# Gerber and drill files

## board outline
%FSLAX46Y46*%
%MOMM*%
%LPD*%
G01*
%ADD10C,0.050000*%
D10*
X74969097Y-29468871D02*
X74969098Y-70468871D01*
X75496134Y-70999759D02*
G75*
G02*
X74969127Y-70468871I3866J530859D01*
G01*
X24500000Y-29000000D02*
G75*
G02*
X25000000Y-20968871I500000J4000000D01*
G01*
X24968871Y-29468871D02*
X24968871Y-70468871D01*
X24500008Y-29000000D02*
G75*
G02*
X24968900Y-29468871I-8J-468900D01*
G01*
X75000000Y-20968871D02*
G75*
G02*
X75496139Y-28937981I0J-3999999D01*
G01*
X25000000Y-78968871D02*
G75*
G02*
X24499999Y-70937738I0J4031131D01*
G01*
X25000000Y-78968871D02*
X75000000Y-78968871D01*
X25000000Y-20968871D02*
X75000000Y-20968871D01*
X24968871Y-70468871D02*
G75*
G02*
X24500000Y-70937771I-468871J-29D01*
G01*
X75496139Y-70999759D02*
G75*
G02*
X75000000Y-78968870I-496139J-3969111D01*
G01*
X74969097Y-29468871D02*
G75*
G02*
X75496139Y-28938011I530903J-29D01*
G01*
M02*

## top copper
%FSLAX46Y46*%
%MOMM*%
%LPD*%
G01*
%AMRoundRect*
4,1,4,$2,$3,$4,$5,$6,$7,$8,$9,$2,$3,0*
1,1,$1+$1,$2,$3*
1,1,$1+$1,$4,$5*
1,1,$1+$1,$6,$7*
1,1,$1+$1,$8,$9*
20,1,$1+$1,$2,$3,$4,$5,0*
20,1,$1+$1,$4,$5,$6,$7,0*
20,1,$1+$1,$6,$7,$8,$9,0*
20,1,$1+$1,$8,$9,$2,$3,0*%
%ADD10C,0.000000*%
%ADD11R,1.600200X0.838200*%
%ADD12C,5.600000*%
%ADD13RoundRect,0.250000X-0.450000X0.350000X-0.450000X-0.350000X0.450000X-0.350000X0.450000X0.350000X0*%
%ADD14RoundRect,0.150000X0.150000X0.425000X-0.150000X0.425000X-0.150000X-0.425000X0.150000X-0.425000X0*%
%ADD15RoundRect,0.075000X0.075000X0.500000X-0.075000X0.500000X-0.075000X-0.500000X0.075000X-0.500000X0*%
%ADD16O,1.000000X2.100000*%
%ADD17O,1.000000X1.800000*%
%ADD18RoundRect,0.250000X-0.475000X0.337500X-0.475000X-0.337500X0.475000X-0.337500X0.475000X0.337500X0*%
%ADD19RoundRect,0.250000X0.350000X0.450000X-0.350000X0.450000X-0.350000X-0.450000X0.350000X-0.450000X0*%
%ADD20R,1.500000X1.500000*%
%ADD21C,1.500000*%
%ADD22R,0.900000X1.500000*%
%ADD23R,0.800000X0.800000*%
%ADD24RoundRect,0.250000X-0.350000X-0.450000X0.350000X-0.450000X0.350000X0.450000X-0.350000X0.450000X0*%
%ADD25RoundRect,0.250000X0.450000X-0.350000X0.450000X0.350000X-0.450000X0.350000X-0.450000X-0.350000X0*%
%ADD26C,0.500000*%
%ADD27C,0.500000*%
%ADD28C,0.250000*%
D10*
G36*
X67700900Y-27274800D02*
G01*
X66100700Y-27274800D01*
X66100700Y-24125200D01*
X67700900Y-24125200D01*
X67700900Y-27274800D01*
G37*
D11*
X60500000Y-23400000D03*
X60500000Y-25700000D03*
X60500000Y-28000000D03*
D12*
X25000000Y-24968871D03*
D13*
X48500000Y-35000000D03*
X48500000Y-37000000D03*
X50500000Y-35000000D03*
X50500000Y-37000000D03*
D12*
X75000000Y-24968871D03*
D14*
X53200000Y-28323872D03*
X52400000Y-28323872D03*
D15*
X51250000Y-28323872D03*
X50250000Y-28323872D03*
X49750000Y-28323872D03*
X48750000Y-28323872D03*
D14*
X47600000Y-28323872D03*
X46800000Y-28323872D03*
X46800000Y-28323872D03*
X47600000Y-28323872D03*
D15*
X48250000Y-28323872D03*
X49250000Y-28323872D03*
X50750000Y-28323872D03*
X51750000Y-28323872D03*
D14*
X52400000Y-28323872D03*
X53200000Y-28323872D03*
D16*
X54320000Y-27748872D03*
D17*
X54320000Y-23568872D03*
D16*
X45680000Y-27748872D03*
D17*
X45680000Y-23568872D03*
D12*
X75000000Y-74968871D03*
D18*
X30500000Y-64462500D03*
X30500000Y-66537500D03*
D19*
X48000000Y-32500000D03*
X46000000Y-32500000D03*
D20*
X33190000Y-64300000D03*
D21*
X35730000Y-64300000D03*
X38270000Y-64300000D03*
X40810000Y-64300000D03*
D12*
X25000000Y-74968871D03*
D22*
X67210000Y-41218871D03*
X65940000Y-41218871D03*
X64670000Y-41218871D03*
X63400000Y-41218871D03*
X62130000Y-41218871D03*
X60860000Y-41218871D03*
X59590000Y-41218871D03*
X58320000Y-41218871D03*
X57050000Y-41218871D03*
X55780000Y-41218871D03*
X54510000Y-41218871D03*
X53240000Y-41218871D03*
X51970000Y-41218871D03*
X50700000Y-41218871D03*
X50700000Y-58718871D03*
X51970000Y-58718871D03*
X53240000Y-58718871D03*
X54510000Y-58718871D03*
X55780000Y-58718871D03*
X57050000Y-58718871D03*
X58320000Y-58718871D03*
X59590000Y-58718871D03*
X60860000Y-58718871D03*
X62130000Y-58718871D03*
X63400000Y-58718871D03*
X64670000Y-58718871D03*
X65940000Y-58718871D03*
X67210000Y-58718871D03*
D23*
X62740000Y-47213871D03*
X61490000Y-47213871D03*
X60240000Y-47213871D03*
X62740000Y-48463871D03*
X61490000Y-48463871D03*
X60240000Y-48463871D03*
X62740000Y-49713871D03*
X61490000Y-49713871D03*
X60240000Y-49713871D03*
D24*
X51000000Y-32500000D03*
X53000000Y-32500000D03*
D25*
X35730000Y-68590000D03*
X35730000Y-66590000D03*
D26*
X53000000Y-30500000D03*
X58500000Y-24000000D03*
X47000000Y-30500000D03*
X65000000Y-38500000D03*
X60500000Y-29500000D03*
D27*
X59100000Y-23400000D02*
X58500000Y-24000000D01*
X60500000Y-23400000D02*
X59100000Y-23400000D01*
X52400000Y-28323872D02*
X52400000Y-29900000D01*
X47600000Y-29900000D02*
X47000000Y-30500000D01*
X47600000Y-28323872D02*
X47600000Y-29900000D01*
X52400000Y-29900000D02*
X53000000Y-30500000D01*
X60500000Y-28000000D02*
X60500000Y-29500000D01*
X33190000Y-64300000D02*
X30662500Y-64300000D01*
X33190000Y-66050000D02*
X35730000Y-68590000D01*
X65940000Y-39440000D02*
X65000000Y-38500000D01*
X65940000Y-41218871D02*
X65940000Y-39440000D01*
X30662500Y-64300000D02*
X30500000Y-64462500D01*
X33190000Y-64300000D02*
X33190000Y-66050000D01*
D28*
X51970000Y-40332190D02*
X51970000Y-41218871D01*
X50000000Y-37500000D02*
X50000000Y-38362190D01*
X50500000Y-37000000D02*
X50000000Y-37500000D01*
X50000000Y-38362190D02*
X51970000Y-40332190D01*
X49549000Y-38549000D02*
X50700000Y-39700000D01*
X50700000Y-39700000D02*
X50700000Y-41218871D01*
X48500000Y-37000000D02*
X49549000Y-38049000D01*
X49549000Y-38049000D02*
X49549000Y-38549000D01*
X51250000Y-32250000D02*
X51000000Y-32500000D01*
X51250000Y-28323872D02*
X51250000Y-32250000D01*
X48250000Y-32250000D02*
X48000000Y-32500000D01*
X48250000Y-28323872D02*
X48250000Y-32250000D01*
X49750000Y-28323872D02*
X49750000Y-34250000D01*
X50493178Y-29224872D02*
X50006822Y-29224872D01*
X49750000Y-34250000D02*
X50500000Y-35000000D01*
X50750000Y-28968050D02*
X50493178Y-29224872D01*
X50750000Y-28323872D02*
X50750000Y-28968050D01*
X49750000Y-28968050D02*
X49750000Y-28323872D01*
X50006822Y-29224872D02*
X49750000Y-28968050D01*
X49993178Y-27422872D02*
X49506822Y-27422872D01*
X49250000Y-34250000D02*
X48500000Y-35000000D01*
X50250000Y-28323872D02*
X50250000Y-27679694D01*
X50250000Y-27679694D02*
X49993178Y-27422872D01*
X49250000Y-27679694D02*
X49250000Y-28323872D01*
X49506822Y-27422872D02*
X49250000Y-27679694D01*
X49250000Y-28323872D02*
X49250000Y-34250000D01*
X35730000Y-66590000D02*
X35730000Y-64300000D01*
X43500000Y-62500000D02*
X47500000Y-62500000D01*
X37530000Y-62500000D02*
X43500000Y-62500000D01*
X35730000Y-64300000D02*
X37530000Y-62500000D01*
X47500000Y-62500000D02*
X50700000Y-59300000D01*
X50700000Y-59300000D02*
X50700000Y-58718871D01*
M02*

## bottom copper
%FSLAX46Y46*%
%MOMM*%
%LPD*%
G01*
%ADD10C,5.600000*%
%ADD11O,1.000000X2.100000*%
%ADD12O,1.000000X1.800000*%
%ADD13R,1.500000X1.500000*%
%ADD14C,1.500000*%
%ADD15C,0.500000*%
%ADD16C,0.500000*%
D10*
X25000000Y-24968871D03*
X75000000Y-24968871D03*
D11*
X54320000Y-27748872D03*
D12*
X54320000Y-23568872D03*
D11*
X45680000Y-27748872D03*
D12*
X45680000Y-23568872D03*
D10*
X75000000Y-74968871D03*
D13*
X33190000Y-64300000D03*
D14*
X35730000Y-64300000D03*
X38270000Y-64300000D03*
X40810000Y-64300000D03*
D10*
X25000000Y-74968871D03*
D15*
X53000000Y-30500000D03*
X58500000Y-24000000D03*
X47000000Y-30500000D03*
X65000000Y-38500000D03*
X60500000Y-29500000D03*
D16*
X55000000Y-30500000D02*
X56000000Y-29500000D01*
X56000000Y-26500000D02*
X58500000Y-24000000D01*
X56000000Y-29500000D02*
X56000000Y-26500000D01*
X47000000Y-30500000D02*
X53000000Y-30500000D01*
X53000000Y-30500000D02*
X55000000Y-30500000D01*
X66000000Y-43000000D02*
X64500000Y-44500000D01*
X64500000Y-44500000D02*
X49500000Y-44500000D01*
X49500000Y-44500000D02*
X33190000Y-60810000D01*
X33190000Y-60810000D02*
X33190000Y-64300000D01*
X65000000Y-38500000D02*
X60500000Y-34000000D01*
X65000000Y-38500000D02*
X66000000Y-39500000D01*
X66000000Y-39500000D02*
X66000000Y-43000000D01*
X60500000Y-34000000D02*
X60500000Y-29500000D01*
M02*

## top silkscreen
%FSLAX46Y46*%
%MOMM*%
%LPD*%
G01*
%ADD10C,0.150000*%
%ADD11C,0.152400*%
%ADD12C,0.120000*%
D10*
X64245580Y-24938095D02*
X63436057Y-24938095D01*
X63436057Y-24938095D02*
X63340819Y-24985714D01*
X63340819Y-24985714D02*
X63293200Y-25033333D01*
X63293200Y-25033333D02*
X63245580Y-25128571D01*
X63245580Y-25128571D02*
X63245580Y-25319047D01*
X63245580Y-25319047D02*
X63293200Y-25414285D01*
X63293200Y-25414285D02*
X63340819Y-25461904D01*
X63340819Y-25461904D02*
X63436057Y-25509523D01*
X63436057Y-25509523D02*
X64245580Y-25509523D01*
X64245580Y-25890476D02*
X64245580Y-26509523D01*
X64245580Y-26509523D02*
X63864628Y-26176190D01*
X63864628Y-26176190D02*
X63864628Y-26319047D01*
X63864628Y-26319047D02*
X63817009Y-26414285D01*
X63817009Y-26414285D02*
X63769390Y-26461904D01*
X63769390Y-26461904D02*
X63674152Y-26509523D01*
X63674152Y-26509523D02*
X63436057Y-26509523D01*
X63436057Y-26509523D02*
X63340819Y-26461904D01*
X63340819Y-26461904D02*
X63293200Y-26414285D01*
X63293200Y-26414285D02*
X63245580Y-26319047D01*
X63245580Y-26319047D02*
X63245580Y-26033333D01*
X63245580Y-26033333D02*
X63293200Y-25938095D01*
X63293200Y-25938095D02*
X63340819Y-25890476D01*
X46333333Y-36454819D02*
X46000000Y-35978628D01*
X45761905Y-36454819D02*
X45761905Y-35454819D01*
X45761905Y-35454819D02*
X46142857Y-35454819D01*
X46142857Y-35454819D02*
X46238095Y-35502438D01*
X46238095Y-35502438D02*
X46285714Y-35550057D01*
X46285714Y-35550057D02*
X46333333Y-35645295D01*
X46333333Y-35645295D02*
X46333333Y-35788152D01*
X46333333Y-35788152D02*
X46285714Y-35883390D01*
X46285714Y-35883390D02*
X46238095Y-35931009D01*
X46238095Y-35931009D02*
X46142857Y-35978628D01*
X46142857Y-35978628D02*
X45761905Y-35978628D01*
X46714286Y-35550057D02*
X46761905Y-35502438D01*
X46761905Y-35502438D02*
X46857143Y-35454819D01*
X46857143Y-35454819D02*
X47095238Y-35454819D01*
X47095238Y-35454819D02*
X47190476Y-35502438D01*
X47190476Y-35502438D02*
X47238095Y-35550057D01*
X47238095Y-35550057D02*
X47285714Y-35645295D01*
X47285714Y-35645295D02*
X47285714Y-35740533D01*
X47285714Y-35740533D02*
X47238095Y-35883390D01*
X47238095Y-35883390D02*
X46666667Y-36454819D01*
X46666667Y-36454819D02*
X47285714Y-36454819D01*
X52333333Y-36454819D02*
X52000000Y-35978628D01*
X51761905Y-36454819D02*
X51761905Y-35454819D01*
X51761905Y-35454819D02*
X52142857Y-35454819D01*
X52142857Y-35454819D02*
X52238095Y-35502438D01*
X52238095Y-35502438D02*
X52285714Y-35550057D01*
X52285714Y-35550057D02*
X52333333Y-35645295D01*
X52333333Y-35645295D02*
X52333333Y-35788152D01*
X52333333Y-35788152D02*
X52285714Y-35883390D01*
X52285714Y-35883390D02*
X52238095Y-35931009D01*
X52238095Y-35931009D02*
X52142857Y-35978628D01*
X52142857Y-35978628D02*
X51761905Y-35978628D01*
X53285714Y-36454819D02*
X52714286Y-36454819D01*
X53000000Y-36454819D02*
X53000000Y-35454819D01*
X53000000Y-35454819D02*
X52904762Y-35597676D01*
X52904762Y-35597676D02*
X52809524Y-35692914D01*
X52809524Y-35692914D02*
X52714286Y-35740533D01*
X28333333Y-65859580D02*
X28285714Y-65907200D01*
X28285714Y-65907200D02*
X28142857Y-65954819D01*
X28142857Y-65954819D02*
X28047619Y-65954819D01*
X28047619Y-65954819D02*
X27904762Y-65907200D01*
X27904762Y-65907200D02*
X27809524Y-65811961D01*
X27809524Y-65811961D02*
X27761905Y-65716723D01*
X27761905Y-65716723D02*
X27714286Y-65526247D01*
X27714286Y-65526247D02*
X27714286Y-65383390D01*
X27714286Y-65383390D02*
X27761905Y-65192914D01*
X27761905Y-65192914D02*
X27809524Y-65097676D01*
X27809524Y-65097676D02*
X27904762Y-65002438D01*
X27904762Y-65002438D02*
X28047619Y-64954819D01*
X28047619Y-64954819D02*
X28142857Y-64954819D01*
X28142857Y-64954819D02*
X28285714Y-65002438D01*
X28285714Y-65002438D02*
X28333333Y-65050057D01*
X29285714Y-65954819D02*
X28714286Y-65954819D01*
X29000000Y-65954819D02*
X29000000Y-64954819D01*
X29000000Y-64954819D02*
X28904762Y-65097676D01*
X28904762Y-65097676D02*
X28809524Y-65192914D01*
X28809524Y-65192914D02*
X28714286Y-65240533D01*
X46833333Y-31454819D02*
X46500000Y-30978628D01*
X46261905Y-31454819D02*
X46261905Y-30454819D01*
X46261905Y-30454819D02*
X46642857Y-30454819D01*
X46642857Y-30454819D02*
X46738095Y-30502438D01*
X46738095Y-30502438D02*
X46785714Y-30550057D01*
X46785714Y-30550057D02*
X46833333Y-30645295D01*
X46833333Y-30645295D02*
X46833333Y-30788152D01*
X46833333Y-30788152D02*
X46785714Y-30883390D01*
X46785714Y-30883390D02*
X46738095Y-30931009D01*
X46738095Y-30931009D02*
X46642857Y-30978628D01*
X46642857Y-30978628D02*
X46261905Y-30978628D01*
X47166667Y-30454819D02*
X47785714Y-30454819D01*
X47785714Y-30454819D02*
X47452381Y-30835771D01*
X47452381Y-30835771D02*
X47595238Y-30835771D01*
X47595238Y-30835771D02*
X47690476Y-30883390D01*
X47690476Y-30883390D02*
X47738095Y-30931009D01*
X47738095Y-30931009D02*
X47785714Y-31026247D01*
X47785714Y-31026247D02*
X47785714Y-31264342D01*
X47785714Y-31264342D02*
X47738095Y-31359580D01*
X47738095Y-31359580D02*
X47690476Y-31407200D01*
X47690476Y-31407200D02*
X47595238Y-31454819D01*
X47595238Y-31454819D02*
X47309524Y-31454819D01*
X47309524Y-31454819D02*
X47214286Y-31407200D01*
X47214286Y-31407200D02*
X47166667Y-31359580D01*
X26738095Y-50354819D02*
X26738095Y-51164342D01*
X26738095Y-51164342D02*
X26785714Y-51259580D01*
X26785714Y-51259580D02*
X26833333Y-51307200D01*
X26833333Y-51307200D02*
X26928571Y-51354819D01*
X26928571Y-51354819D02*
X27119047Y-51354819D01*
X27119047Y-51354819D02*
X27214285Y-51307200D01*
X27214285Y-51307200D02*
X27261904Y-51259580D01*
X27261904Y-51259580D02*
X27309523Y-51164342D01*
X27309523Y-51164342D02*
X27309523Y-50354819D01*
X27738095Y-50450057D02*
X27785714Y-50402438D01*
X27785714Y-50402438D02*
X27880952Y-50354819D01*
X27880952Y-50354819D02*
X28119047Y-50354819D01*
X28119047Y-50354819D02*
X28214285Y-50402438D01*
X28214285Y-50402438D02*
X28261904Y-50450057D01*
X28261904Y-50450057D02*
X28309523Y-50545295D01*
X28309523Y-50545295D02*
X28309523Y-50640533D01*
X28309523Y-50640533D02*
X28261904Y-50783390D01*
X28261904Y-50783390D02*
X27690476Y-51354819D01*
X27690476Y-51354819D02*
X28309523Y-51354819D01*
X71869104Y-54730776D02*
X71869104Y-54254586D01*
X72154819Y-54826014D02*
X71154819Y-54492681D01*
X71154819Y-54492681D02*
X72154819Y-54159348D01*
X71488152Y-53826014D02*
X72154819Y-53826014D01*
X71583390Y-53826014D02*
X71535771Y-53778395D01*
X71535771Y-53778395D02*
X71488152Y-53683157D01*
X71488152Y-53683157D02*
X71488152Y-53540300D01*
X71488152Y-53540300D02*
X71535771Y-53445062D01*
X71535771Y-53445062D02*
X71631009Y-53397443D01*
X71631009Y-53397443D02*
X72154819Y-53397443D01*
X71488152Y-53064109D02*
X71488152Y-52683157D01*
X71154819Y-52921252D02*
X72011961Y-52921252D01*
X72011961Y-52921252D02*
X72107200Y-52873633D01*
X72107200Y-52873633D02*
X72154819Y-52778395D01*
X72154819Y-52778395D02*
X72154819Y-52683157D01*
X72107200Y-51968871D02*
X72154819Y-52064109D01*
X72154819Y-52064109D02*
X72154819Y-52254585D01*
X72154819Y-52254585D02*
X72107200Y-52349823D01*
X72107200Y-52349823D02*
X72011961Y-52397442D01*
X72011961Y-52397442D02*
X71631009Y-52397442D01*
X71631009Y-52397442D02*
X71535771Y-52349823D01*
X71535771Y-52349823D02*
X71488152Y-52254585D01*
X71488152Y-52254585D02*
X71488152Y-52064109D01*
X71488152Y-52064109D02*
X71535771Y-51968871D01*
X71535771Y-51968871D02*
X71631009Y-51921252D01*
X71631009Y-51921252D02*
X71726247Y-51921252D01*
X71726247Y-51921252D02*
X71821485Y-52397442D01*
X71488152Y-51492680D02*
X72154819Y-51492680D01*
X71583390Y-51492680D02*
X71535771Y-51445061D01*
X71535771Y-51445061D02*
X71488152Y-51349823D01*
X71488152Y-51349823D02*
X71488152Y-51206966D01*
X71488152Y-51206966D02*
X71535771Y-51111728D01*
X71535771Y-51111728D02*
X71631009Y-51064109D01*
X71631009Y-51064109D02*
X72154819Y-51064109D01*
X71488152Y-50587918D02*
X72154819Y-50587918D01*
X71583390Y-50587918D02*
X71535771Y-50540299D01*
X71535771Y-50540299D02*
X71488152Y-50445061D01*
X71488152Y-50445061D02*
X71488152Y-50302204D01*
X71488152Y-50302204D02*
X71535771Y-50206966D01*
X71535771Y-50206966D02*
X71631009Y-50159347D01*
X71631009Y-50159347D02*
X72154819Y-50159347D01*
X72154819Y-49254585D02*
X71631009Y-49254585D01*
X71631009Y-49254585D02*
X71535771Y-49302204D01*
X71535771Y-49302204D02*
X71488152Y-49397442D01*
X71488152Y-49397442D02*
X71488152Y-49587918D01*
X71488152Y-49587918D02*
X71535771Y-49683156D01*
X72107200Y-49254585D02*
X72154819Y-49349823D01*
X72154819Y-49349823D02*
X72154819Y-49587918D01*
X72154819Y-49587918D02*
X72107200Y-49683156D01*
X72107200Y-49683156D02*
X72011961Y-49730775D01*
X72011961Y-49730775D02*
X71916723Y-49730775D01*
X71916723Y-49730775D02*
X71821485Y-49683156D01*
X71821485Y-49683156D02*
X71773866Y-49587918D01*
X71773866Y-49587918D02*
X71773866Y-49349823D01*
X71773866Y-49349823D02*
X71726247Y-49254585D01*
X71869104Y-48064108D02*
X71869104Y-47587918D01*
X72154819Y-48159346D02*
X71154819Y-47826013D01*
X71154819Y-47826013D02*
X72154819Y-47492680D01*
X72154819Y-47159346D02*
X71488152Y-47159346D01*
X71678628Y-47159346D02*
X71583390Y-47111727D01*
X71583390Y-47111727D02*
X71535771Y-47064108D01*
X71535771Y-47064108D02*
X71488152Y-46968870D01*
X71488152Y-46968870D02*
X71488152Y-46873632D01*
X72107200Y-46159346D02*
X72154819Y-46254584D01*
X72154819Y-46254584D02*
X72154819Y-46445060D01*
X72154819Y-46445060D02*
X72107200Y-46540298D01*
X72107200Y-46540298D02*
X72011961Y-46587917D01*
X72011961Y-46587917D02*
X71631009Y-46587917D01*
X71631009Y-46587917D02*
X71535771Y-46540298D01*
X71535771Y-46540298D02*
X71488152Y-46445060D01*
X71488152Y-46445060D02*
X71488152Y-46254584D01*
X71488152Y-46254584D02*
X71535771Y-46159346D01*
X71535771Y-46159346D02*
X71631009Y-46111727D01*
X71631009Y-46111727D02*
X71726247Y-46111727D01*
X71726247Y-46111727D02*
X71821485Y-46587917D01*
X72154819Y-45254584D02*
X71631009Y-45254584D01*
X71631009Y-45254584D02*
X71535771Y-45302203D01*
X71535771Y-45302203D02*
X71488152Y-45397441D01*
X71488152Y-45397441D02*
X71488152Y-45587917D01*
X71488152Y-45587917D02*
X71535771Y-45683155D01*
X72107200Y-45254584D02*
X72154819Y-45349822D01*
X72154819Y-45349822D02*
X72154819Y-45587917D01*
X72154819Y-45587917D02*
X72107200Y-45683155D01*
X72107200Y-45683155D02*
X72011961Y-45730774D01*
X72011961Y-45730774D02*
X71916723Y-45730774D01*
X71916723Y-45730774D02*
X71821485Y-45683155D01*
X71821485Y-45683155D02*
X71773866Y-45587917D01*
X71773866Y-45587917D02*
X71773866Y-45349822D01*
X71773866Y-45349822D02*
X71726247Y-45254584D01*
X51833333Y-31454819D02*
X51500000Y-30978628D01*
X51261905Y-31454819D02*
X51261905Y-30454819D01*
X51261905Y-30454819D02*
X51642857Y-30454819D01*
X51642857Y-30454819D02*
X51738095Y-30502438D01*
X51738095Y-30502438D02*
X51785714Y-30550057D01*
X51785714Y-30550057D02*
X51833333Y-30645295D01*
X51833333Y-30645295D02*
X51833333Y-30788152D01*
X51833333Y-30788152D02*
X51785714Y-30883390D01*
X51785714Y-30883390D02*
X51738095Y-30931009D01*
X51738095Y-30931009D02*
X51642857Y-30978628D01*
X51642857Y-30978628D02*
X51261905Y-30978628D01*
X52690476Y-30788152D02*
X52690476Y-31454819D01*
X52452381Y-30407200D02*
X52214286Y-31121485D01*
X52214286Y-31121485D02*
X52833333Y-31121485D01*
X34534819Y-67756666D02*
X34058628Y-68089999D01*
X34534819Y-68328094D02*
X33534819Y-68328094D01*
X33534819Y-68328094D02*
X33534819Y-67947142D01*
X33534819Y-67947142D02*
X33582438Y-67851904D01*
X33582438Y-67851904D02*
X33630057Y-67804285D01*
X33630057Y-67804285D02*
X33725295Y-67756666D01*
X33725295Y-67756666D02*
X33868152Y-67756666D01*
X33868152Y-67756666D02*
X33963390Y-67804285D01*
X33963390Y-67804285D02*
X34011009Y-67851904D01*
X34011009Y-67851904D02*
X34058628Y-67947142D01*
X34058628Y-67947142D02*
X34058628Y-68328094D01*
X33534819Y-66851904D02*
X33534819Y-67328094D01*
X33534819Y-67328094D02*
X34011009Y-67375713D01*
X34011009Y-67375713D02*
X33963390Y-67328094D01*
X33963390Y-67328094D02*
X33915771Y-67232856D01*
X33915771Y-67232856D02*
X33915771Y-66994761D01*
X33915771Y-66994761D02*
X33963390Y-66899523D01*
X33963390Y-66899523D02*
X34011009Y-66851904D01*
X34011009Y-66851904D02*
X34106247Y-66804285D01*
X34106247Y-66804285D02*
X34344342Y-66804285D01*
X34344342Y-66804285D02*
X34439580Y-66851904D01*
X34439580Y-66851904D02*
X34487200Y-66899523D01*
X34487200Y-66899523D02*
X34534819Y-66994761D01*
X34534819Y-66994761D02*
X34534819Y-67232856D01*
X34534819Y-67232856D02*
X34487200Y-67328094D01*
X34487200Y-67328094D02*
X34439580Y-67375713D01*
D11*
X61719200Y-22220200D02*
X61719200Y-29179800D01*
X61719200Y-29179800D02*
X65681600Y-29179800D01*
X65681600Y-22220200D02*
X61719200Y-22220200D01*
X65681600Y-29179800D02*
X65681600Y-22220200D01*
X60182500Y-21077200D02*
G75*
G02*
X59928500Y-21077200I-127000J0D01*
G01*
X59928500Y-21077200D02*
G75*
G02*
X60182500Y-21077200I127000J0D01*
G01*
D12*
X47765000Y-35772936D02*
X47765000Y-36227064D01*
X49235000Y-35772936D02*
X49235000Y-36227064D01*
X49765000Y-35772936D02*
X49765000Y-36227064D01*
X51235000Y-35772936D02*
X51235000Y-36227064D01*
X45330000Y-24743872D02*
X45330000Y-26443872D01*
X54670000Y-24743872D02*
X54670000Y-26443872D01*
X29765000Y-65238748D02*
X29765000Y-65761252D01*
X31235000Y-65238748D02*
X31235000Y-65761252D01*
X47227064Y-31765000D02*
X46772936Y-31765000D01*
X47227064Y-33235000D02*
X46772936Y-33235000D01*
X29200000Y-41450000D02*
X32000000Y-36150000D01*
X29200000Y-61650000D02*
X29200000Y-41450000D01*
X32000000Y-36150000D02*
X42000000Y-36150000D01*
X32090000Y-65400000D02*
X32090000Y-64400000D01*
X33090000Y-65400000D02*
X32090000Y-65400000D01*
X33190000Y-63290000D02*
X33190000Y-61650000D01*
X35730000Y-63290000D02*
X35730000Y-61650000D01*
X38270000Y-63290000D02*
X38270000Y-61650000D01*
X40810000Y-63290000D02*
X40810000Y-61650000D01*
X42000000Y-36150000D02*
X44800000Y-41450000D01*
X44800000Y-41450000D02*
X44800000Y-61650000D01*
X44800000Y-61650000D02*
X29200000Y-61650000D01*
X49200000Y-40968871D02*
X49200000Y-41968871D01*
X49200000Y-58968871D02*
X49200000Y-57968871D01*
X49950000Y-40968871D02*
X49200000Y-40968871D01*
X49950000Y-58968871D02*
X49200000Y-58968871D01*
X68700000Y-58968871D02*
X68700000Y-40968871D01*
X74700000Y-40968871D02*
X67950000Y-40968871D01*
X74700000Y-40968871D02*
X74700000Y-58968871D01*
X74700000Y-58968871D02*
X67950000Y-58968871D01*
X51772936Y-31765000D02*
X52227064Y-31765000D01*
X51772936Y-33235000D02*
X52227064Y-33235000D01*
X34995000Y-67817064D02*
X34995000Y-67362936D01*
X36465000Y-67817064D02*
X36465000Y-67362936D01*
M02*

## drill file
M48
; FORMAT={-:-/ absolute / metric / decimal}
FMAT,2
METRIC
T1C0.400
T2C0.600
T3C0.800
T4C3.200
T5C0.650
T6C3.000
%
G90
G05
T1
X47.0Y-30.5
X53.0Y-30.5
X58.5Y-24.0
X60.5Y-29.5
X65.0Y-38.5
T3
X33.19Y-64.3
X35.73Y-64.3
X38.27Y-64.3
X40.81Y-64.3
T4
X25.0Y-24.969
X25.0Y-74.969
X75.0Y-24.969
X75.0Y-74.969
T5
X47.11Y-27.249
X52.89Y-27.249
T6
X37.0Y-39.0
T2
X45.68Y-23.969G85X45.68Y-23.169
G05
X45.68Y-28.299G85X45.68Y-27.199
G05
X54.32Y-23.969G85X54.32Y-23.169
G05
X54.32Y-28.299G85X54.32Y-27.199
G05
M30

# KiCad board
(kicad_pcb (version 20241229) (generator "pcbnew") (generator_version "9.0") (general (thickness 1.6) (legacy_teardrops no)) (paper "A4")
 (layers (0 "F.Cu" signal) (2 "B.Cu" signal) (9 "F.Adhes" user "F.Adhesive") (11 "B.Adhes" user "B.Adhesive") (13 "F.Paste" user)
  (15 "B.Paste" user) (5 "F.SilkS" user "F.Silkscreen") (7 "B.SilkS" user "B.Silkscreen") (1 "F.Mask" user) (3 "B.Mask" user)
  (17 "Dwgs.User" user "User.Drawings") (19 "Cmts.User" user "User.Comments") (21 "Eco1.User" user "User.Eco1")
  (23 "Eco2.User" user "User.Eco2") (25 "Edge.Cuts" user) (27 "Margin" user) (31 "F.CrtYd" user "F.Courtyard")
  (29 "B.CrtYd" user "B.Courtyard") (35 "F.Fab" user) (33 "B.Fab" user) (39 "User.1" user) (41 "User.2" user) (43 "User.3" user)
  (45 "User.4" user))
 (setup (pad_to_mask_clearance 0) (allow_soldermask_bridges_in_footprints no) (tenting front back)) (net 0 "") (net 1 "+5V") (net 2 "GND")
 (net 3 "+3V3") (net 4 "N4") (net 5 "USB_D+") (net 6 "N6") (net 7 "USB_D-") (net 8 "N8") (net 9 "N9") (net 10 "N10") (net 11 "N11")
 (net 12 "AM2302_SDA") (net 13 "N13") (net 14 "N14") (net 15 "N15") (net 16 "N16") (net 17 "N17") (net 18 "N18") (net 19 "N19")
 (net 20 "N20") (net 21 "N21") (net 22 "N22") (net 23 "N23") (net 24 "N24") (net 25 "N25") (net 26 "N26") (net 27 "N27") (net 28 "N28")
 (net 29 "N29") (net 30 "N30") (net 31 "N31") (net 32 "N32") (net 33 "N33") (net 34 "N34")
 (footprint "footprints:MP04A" (layer "F.Cu") (at 63.7004 25.7 -90)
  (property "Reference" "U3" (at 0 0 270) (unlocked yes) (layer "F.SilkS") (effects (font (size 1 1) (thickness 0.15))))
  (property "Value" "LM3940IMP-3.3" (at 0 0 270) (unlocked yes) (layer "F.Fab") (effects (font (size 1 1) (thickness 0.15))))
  (fp_poly
   (pts (xy 1.5748 -4.0005) (xy -1.5748 -4.0005) (xy -1.5748 -2.4003) (xy 1.5748 -2.4003)) (stroke (width 0) (type solid)) (fill yes)
   (layer "F.Cu"))
  (fp_line (start -3.4798 1.9812) (end 3.4798 1.9812) (stroke (width 0.1524) (type solid)) (layer "F.SilkS"))
  (fp_line (start 3.4798 1.9812) (end 3.4798 -1.9812) (stroke (width 0.1524) (type solid)) (layer "F.SilkS"))
  (fp_line (start -3.4798 -1.9812) (end -3.4798 1.9812) (stroke (width 0.1524) (type solid)) (layer "F.SilkS"))
  (fp_line (start 3.4798 -1.9812) (end -3.4798 -1.9812) (stroke (width 0.1524) (type solid)) (layer "F.SilkS"))
  (fp_circle (center -4.6228 3.6449) (end -4.4958 3.6449) (stroke (width 0.1524) (type solid)) (fill no) (layer "F.SilkS"))
  (pad "1" smd rect (at -2.3 3.2004 270) (size 0.8382 1.6002) (layers "F.Cu" "F.Mask" "F.Paste") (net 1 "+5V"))
  (pad "2" smd rect (at 0 3.2004 270) (size 0.8382 1.6002) (layers "F.Cu" "F.Mask" "F.Paste") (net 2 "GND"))
  (pad "3" smd rect (at 2.3 3.2004 270) (size 0.8382 1.6002) (layers "F.Cu" "F.Mask" "F.Paste") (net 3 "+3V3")))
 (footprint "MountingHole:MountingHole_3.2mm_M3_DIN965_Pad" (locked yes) (layer "F.Cu") (at 25 24.968871)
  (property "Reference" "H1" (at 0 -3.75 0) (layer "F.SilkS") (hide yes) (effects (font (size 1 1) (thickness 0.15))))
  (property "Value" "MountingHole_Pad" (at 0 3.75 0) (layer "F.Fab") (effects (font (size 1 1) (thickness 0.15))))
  (pad "1" thru_hole circle (at 0 0) (size 5.6 5.6) (drill 3.2) (layers "*.Cu" "*.Mask") (remove_unused_layers no) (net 2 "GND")
   (zone_connect 2)))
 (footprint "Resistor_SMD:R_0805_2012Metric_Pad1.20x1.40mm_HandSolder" (layer "F.Cu") (at 48.5 36 -90)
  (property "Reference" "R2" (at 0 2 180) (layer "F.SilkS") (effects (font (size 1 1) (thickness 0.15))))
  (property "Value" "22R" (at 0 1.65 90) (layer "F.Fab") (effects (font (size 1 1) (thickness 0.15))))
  (fp_line (start -0.227064 0.735) (end 0.227064 0.735) (stroke (width 0.12) (type solid)) (layer "F.SilkS"))
  (fp_line (start -0.227064 -0.735) (end 0.227064 -0.735) (stroke (width 0.12) (type solid)) (layer "F.SilkS"))
  (pad "1" smd roundrect (at -1 0 270) (size 1.2 1.4) (layers "F.Cu" "F.Mask" "F.Paste") (roundrect_rratio 0.208333) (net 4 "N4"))
  (pad "2" smd roundrect (at 1 0 270) (size 1.2 1.4) (layers "F.Cu" "F.Mask" "F.Paste") (roundrect_rratio 0.208333) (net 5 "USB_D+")))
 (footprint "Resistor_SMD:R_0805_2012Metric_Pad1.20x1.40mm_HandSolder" (layer "F.Cu") (at 50.5 36 -90)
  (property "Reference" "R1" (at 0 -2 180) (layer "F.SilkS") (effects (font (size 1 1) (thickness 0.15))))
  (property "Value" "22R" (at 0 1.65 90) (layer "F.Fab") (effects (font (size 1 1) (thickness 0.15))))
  (fp_line (start -0.227064 0.735) (end 0.227064 0.735) (stroke (width 0.12) (type solid)) (layer "F.SilkS"))
  (fp_line (start -0.227064 -0.735) (end 0.227064 -0.735) (stroke (width 0.12) (type solid)) (layer "F.SilkS"))
  (pad "1" smd roundrect (at -1 0 270) (size 1.2 1.4) (layers "F.Cu" "F.Mask" "F.Paste") (roundrect_rratio 0.208333) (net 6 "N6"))
  (pad "2" smd roundrect (at 1 0 270) (size 1.2 1.4) (layers "F.Cu" "F.Mask" "F.Paste") (roundrect_rratio 0.208333) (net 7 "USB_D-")))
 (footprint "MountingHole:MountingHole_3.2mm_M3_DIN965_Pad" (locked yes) (layer "F.Cu") (at 75 24.968871)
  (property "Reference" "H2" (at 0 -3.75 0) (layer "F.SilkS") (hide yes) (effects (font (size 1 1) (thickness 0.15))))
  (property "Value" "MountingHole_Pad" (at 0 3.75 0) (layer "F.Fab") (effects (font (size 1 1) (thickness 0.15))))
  (pad "1" thru_hole circle (at 0 0) (size 5.6 5.6) (drill 3.2) (layers "*.Cu" "*.Mask") (remove_unused_layers no) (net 2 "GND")
   (zone_connect 2)))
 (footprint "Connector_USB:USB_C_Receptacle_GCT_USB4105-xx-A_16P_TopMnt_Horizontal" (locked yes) (layer "F.Cu") (at 50 24.643872 180)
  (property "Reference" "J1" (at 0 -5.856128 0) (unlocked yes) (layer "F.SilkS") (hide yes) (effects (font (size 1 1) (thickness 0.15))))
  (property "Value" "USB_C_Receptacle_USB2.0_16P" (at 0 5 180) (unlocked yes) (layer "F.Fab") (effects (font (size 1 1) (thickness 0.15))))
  (fp_line (start 4.67 -0.1) (end 4.67 -1.8) (stroke (width 0.12) (type solid)) (layer "F.SilkS"))
  (fp_line (start -4.67 -0.1) (end -4.67 -1.8) (stroke (width 0.12) (type solid)) (layer "F.SilkS"))
  (pad "" np_thru_hole circle (at -2.89 -2.605 180) (size 0.65 0.65) (drill 0.65) (layers "*.Cu" "*.Mask"))
  (pad "" np_thru_hole circle (at 2.89 -2.605 180) (size 0.65 0.65) (drill 0.65) (layers "*.Cu" "*.Mask"))
  (pad "A1" smd roundrect (at -3.2 -3.68 180) (size 0.6 1.15) (layers "F.Cu" "F.Mask" "F.Paste") (roundrect_rratio 0.25) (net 2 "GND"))
  (pad "A4" smd roundrect (at -2.4 -3.68 180) (size 0.6 1.15) (layers "F.Cu" "F.Mask" "F.Paste") (roundrect_rratio 0.25) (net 1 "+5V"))
  (pad "A5" smd roundrect (at -1.25 -3.68 180) (size 0.3 1.15) (layers "F.Cu" "F.Mask" "F.Paste") (roundrect_rratio 0.25) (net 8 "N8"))
  (pad "A6" smd roundrect (at -0.25 -3.68 180) (size 0.3 1.15) (layers "F.Cu" "F.Mask" "F.Paste") (roundrect_rratio 0.25) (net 4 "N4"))
  (pad "A7" smd roundrect (at 0.25 -3.68 180) (size 0.3 1.15) (layers "F.Cu" "F.Mask" "F.Paste") (roundrect_rratio 0.25) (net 6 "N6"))
  (pad "A8" smd roundrect (at 1.25 -3.68 180) (size 0.3 1.15) (layers "F.Cu" "F.Mask" "F.Paste") (roundrect_rratio 0.25) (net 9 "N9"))
  (pad "A9" smd roundrect (at 2.4 -3.68 180) (size 0.6 1.15) (layers "F.Cu" "F.Mask" "F.Paste") (roundrect_rratio 0.25) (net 1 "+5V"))
  (pad "A12" smd roundrect (at 3.2 -3.68 180) (size 0.6 1.15) (layers "F.Cu" "F.Mask" "F.Paste") (roundrect_rratio 0.25) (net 2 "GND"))
  (pad "B1" smd roundrect (at 3.2 -3.68 180) (size 0.6 1.15) (layers "F.Cu" "F.Mask" "F.Paste") (roundrect_rratio 0.25) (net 2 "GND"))
  (pad "B4" smd roundrect (at 2.4 -3.68 180) (size 0.6 1.15) (layers "F.Cu" "F.Mask" "F.Paste") (roundrect_rratio 0.25) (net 1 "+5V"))
  (pad "B5" smd roundrect (at 1.75 -3.68 180) (size 0.3 1.15) (layers "F.Cu" "F.Mask" "F.Paste") (roundrect_rratio 0.25) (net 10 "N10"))
  (pad "B6" smd roundrect (at 0.75 -3.68 180) (size 0.3 1.15) (layers "F.Cu" "F.Mask" "F.Paste") (roundrect_rratio 0.25) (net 4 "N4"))
  (pad "B7" smd roundrect (at -0.75 -3.68 180) (size 0.3 1.15) (layers "F.Cu" "F.Mask" "F.Paste") (roundrect_rratio 0.25) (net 6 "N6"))
  (pad "B8" smd roundrect (at -1.75 -3.68 180) (size 0.3 1.15) (layers "F.Cu" "F.Mask" "F.Paste") (roundrect_rratio 0.25) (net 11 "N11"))
  (pad "B9" smd roundrect (at -2.4 -3.68 180) (size 0.6 1.15) (layers "F.Cu" "F.Mask" "F.Paste") (roundrect_rratio 0.25) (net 1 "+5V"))
  (pad "B12" smd roundrect (at -3.2 -3.68 180) (size 0.6 1.15) (layers "F.Cu" "F.Mask" "F.Paste") (roundrect_rratio 0.25) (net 2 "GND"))
  (pad "S1" thru_hole oval (at -4.32 -3.105 180) (size 1 2.1) (drill oval 0.6 1.7) (layers "*.Cu" "*.Mask" "F.Paste")
   (remove_unused_layers no) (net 2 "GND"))
  (pad "S1" thru_hole oval (at -4.32 1.075 180) (size 1 1.8) (drill oval 0.6 1.4) (layers "*.Cu" "*.Mask" "F.Paste")
   (remove_unused_layers no) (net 2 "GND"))
  (pad "S1" thru_hole oval (at 4.32 -3.105 180) (size 1 2.1) (drill oval 0.6 1.7) (layers "*.Cu" "*.Mask" "F.Paste")
   (remove_unused_layers no) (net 2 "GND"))
  (pad "S1" thru_hole oval (at 4.32 1.075 180) (size 1 1.8) (drill oval 0.6 1.4) (layers "*.Cu" "*.Mask" "F.Paste")
   (remove_unused_layers no) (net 2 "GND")))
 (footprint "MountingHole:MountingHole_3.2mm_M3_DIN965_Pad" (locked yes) (layer "F.Cu") (at 75 74.968871)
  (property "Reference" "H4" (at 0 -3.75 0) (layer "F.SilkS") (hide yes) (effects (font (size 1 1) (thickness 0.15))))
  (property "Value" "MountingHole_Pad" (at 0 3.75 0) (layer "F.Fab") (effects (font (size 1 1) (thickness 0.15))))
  (pad "1" thru_hole circle (at 0 0) (size 5.6 5.6) (drill 3.2) (layers "*.Cu" "*.Mask") (remove_unused_layers no) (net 2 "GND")
   (zone_connect 2)))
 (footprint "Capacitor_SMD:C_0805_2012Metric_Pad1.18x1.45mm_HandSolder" (layer "F.Cu") (at 30.5 65.5 -90)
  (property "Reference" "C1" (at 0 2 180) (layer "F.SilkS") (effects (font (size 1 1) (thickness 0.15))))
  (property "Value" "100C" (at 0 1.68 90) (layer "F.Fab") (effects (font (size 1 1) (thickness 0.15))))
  (fp_line (start -0.261252 0.735) (end 0.261252 0.735) (stroke (width 0.12) (type solid)) (layer "F.SilkS"))
  (fp_line (start -0.261252 -0.735) (end 0.261252 -0.735) (stroke (width 0.12) (type solid)) (layer "F.SilkS"))
  (pad "1" smd roundrect (at -1.0375 0 270) (size 1.175 1.45) (layers "F.Cu" "F.Mask" "F.Paste") (roundrect_rratio 0.212766) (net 3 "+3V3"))
  (pad "2" smd roundrect (at 1.0375 0 270) (size 1.175 1.45) (layers "F.Cu" "F.Mask" "F.Paste") (roundrect_rratio 0.212766) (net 2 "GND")))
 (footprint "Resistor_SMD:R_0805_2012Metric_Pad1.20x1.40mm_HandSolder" (layer "F.Cu") (at 47 32.5 180)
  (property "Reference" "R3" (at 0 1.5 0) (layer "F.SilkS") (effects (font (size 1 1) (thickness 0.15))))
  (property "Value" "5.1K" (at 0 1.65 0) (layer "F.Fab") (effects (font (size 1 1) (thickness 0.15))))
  (fp_line (start -0.227064 0.735) (end 0.227064 0.735) (stroke (width 0.12) (type solid)) (layer "F.SilkS"))
  (fp_line (start -0.227064 -0.735) (end 0.227064 -0.735) (stroke (width 0.12) (type solid)) (layer "F.SilkS"))
  (pad "1" smd roundrect (at -1 0 180) (size 1.2 1.4) (layers "F.Cu" "F.Mask" "F.Paste") (roundrect_rratio 0.208333) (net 10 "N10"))
  (pad "2" smd roundrect (at 1 0 180) (size 1.2 1.4) (layers "F.Cu" "F.Mask" "F.Paste") (roundrect_rratio 0.208333) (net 2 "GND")))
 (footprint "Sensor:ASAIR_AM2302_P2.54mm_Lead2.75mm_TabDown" (layer "F.Cu") (at 33.19 64.3 90)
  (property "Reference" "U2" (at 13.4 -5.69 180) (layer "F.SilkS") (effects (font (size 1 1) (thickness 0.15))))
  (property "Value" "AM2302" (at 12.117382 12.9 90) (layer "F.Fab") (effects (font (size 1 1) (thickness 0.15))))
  (fp_line (start 22.85 -3.99) (end 28.15 -1.19) (stroke (width 0.12) (type default)) (layer "F.SilkS"))
  (fp_line (start 2.65 -3.99) (end 22.85 -3.99) (stroke (width 0.12) (type solid)) (layer "F.SilkS"))
  (fp_line (start 28.15 -1.19) (end 28.15 8.81) (stroke (width 0.12) (type solid)) (layer "F.SilkS"))
  (fp_line (start -1.1 -1.1) (end -0.1 -1.1) (stroke (width 0.12) (type default)) (layer "F.SilkS"))
  (fp_line (start -1.1 -0.1) (end -1.1 -1.1) (stroke (width 0.12) (type default)) (layer "F.SilkS"))
  (fp_line (start 1.01 0) (end 2.65 0) (stroke (width 0.12) (type default)) (layer "F.SilkS"))
  (fp_line (start 1.01 2.54) (end 2.65 2.54) (stroke (width 0.12) (type default)) (layer "F.SilkS"))
  (fp_line (start 1.01 5.08) (end 2.65 5.08) (stroke (width 0.12) (type default)) (layer "F.SilkS"))
  (fp_line (start 1.01 7.62) (end 2.65 7.62) (stroke (width 0.12) (type default)) (layer "F.SilkS"))
  (fp_line (start 28.15 8.81) (end 22.85 11.61) (stroke (width 0.12) (type default)) (layer "F.SilkS"))
  (fp_line (start 22.85 11.61) (end 2.65 11.61) (stroke (width 0.12) (type solid)) (layer "F.SilkS"))
  (fp_line (start 2.65 11.61) (end 2.65 -3.99) (stroke (width 0.12) (type solid)) (layer "F.SilkS"))
  (pad "" np_thru_hole circle (at 25.3 3.81 90) (size 3 3) (drill 3) (layers "*.Cu" "*.Mask"))
  (pad "1" thru_hole rect (at 0 0 90) (size 1.5 1.5) (drill 0.8) (layers "*.Cu" "*.Mask") (remove_unused_layers no) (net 3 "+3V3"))
  (pad "2" thru_hole circle (at 0 2.54 90) (size 1.5 1.5) (drill 0.8) (layers "*.Cu" "*.Mask") (remove_unused_layers no)
   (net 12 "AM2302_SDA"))
  (pad "3" thru_hole circle (at 0 5.08 90) (size 1.5 1.5) (drill 0.8) (layers "*.Cu" "*.Mask") (remove_unused_layers no) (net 2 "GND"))
  (pad "4" thru_hole circle (at 0 7.62 90) (size 1.5 1.5) (drill 0.8) (layers "*.Cu" "*.Mask") (remove_unused_layers no) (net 2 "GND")))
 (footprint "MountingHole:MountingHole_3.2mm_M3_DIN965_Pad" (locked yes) (layer "F.Cu") (at 25 74.968871)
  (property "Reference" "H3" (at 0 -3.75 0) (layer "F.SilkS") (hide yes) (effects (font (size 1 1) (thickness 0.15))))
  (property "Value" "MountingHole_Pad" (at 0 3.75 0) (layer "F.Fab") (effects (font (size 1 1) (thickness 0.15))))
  (pad "1" thru_hole circle (at 0 0) (size 5.6 5.6) (drill 3.2) (layers "*.Cu" "*.Mask") (remove_unused_layers no) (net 2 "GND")
   (zone_connect 2)))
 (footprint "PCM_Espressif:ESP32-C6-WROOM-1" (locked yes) (layer "F.Cu") (at 58.95 49.968871 -90)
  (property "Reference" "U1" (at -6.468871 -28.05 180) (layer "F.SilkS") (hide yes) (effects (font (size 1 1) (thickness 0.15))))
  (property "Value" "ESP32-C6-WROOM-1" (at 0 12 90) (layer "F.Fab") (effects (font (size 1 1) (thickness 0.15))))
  (fp_line (start -9 9.75) (end -8 9.75) (stroke (width 0.12) (type solid)) (layer "F.SilkS"))
  (fp_line (start 9 9.75) (end 8 9.75) (stroke (width 0.12) (type solid)) (layer "F.SilkS"))
  (fp_line (start -9 9) (end -9 9.75) (stroke (width 0.12) (type solid)) (layer "F.SilkS"))
  (fp_line (start 9 9) (end 9 9.75) (stroke (width 0.12) (type solid)) (layer "F.SilkS"))
  (fp_line (start 9 -9.75) (end -9 -9.75) (stroke (width 0.12) (type solid)) (layer "F.SilkS"))
  (fp_line (start -9 -15.75) (end -9 -9) (stroke (width 0.12) (type solid)) (layer "F.SilkS"))
  (fp_line (start -9 -15.75) (end 9 -15.75) (stroke (width 0.12) (type solid)) (layer "F.SilkS"))
  (fp_line (start 9 -15.75) (end 9 -9) (stroke (width 0.12) (type solid)) (layer "F.SilkS"))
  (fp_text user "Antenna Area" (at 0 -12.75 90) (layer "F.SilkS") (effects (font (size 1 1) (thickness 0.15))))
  (pad "1" smd rect (at -8.75 -8.26 270) (size 1.5 0.9) (layers "F.Cu" "F.Mask" "F.Paste") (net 2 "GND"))
  (pad "2" smd rect (at -8.75 -6.99 270) (size 1.5 0.9) (layers "F.Cu" "F.Mask" "F.Paste") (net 3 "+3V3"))
  (pad "3" smd rect (at -8.75 -5.72 270) (size 1.5 0.9) (layers "F.Cu" "F.Mask" "F.Paste") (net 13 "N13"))
  (pad "4" smd rect (at -8.75 -4.45 270) (size 1.5 0.9) (layers "F.Cu" "F.Mask" "F.Paste") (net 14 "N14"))
  (pad "5" smd rect (at -8.75 -3.18 270) (size 1.5 0.9) (layers "F.Cu" "F.Mask" "F.Paste") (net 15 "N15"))
  (pad "6" smd rect (at -8.75 -1.91 270) (size 1.5 0.9) (layers "F.Cu" "F.Mask" "F.Paste") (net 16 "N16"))
  (pad "7" smd rect (at -8.75 -0.64 270) (size 1.5 0.9) (layers "F.Cu" "F.Mask" "F.Paste") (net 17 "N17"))
  (pad "8" smd rect (at -8.75 0.63 270) (size 1.5 0.9) (layers "F.Cu" "F.Mask" "F.Paste") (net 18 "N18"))
  (pad "9" smd rect (at -8.75 1.9 270) (size 1.5 0.9) (layers "F.Cu" "F.Mask" "F.Paste") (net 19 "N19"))
  (pad "10" smd rect (at -8.75 3.17 270) (size 1.5 0.9) (layers "F.Cu" "F.Mask" "F.Paste") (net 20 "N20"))
  (pad "11" smd rect (at -8.75 4.44 270) (size 1.5 0.9) (layers "F.Cu" "F.Mask" "F.Paste") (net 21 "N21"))
  (pad "12" smd rect (at -8.75 5.71 270) (size 1.5 0.9) (layers "F.Cu" "F.Mask" "F.Paste") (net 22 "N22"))
  (pad "13" smd rect (at -8.75 6.98 270) (size 1.5 0.9) (layers "F.Cu" "F.Mask" "F.Paste") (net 7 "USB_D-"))
  (pad "14" smd rect (at -8.75 8.25 270) (size 1.5 0.9) (layers "F.Cu" "F.Mask" "F.Paste") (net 5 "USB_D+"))
  (pad "15" smd rect (at 8.75 8.25 90) (size 1.5 0.9) (layers "F.Cu" "F.Mask" "F.Paste") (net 12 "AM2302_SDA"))
  (pad "16" smd rect (at 8.75 6.98 90) (size 1.5 0.9) (layers "F.Cu" "F.Mask" "F.Paste") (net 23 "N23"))
  (pad "17" smd rect (at 8.75 5.71 90) (size 1.5 0.9) (layers "F.Cu" "F.Mask" "F.Paste") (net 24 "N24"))
  (pad "18" smd rect (at 8.75 4.44 90) (size 1.5 0.9) (layers "F.Cu" "F.Mask" "F.Paste") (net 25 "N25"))
  (pad "19" smd rect (at 8.75 3.17 90) (size 1.5 0.9) (layers "F.Cu" "F.Mask" "F.Paste") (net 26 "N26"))
  (pad "20" smd rect (at 8.75 1.9 90) (size 1.5 0.9) (layers "F.Cu" "F.Mask" "F.Paste") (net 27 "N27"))
  (pad "21" smd rect (at 8.75 0.63 90) (size 1.5 0.9) (layers "F.Cu" "F.Mask" "F.Paste") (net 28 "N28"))
  (pad "22" smd rect (at 8.75 -0.64 90) (size 1.5 0.9) (layers "F.Cu" "F.Mask" "F.Paste") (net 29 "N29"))
  (pad "23" smd rect (at 8.75 -1.91 90) (size 1.5 0.9) (layers "F.Cu" "F.Mask" "F.Paste") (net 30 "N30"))
  (pad "24" smd rect (at 8.75 -3.18 90) (size 1.5 0.9) (layers "F.Cu" "F.Mask" "F.Paste") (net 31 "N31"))
  (pad "25" smd rect (at 8.75 -4.45 90) (size 1.5 0.9) (layers "F.Cu" "F.Mask" "F.Paste") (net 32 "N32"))
  (pad "26" smd rect (at 8.75 -5.72 90) (size 1.5 0.9) (layers "F.Cu" "F.Mask" "F.Paste") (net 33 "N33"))
  (pad "27" smd rect (at 8.75 -6.99 90) (size 1.5 0.9) (layers "F.Cu" "F.Mask" "F.Paste") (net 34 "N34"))
  (pad "28" smd rect (at 8.75 -8.26 90) (size 1.5 0.9) (layers "F.Cu" "F.Mask" "F.Paste") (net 2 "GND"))
  (pad "29" smd rect (at -2.755 -3.79 90) (size 0.8 0.8) (layers "F.Cu" "F.Mask" "F.Paste") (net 2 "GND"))
  (pad "29" smd rect (at -2.755 -2.54 90) (size 0.8 0.8) (layers "F.Cu" "F.Mask" "F.Paste") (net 2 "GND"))
  (pad "29" smd rect (at -2.755 -1.29 90) (size 0.8 0.8) (layers "F.Cu" "F.Mask" "F.Paste") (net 2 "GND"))
  (pad "29" smd rect (at -1.505 -3.79 90) (size 0.8 0.8) (layers "F.Cu" "F.Mask" "F.Paste") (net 2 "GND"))
  (pad "29" smd rect (at -1.505 -2.54 90) (size 0.8 0.8) (layers "F.Cu" "F.Mask" "F.Paste") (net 2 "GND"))
  (pad "29" smd rect (at -1.505 -1.29 90) (size 0.8 0.8) (layers "F.Cu" "F.Mask" "F.Paste") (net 2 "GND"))
  (pad "29" smd rect (at -0.255 -3.79 90) (size 0.8 0.8) (layers "F.Cu" "F.Mask" "F.Paste") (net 2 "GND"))
  (pad "29" smd rect (at -0.255 -2.54 90) (size 0.8 0.8) (layers "F.Cu" "F.Mask" "F.Paste") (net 2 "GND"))
  (pad "29" smd rect (at -0.255 -1.29 90) (size 0.8 0.8) (layers "F.Cu" "F.Mask" "F.Paste") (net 2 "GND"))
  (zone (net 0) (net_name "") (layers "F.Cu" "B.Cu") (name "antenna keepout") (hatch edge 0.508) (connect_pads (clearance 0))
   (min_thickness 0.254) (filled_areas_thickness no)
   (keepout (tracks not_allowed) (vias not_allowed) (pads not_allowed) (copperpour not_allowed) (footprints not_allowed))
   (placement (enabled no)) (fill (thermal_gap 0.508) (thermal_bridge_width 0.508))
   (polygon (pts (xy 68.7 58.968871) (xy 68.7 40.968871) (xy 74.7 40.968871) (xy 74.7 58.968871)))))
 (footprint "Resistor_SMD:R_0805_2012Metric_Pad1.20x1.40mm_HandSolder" (layer "F.Cu") (at 52 32.5)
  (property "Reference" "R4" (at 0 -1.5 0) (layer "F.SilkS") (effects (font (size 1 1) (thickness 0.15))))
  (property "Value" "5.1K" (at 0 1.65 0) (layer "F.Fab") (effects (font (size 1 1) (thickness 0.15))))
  (fp_line (start -0.227064 -0.735) (end 0.227064 -0.735) (stroke (width 0.12) (type solid)) (layer "F.SilkS"))
  (fp_line (start -0.227064 0.735) (end 0.227064 0.735) (stroke (width 0.12) (type solid)) (layer "F.SilkS"))
  (pad "1" smd roundrect (at -1 0) (size 1.2 1.4) (layers "F.Cu" "F.Mask" "F.Paste") (roundrect_rratio 0.208333) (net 8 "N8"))
  (pad "2" smd roundrect (at 1 0) (size 1.2 1.4) (layers "F.Cu" "F.Mask" "F.Paste") (roundrect_rratio 0.208333) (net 2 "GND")))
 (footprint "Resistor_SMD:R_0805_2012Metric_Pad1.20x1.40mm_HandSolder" (layer "F.Cu") (at 35.73 67.59 90)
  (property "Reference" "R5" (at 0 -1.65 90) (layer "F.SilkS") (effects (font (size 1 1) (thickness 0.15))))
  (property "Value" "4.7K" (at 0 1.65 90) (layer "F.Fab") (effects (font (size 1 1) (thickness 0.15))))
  (fp_line (start -0.227064 -0.735) (end 0.227064 -0.735) (stroke (width 0.12) (type solid)) (layer "F.SilkS"))
  (fp_line (start -0.227064 0.735) (end 0.227064 0.735) (stroke (width 0.12) (type solid)) (layer "F.SilkS"))
  (pad "1" smd roundrect (at -1 0 90) (size 1.2 1.4) (layers "F.Cu" "F.Mask" "F.Paste") (roundrect_rratio 0.208333) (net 3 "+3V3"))
  (pad "2" smd roundrect (at 1 0 90) (size 1.2 1.4) (layers "F.Cu" "F.Mask" "F.Paste") (roundrect_rratio 0.208333) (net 12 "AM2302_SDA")))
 (gr_line (start 74.969097 29.468871) (end 74.969098 70.468871) (stroke (width 0.05) (type default)) (locked yes) (layer "Edge.Cuts"))
 (gr_arc (start 75.496134 70.999759) (mid 75.123231 70.842906) (end 74.969098 70.468871) (stroke (width 0.05) (type default)) (locked yes)
  (layer "Edge.Cuts"))
 (gr_arc (start 24.5 29) (mid 20.976661 24.749516) (end 25 20.968871) (stroke (width 0.05) (type default)) (locked yes) (layer "Edge.Cuts"))
 (gr_line (start 24.968871 29.468871) (end 24.968871 70.468871) (stroke (width 0.05) (type default)) (locked yes) (layer "Edge.Cuts"))
 (gr_arc (start 24.500008 29) (mid 24.831545 29.137332) (end 24.968871 29.468871) (stroke (width 0.05) (type default)) (locked yes)
  (layer "Edge.Cuts"))
 (gr_arc (start 75 20.968871) (mid 78.99227 24.720321) (end 75.496139 28.937983) (stroke (width 0.05) (type default)) (locked yes)
  (layer "Edge.Cuts"))
 (gr_arc (start 25 78.968871) (mid 20.976661 75.188226) (end 24.5 70.937742) (stroke (width 0.05) (type default)) (locked yes)
  (layer "Edge.Cuts"))
 (gr_line (start 25 78.968871) (end 75 78.968871) (stroke (width 0.05) (type default)) (locked yes) (layer "Edge.Cuts"))
 (gr_line (start 25 20.968871) (end 75 20.968871) (stroke (width 0.05) (type default)) (locked yes) (layer "Edge.Cuts"))
 (gr_arc (start 24.968871 70.468871) (mid 24.831542 70.800413) (end 24.5 70.937742) (stroke (width 0.05) (type default)) (locked yes)
  (layer "Edge.Cuts"))
 (gr_arc (start 75.496139 70.999759) (mid 78.992271 75.217421) (end 75 78.968871) (stroke (width 0.05) (type default)) (locked yes)
  (layer "Edge.Cuts"))
 (gr_arc (start 74.969097 29.468871) (mid 75.123232 29.094833) (end 75.496139 28.937982) (stroke (width 0.05) (type default)) (locked yes)
  (layer "Edge.Cuts"))
 (segment (start 59.1 23.4) (end 58.5 24) (width 0.5) (layer "F.Cu") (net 1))
 (segment (start 60.5 23.4) (end 59.1 23.4) (width 0.5) (layer "F.Cu") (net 1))
 (segment (start 52.4 28.323872) (end 52.4 29.9) (width 0.5) (layer "F.Cu") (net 1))
 (segment (start 47.6 29.9) (end 47 30.5) (width 0.5) (layer "F.Cu") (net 1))
 (segment (start 47.6 28.323872) (end 47.6 29.9) (width 0.5) (layer "F.Cu") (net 1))
 (segment (start 52.4 29.9) (end 53 30.5) (width 0.5) (layer "F.Cu") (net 1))
 (via (at 53 30.5) (size 0.5) (drill 0.4) (layers "F.Cu" "B.Cu") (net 1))
 (via (at 58.5 24) (size 0.5) (drill 0.4) (layers "F.Cu" "B.Cu") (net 1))
 (via (at 47 30.5) (size 0.5) (drill 0.4) (layers "F.Cu" "B.Cu") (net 1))
 (segment (start 55 30.5) (end 56 29.5) (width 0.5) (layer "B.Cu") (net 1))
 (segment (start 56 26.5) (end 58.5 24) (width 0.5) (layer "B.Cu") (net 1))
 (segment (start 56 29.5) (end 56 26.5) (width 0.5) (layer "B.Cu") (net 1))
 (segment (start 47 30.5) (end 53 30.5) (width 0.5) (layer "B.Cu") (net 1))
 (segment (start 53 30.5) (end 55 30.5) (width 0.5) (layer "B.Cu") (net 1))
 (segment (start 60.5 28) (end 60.5 29.5) (width 0.5) (layer "F.Cu") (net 3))
 (segment (start 33.19 64.3) (end 30.6625 64.3) (width 0.5) (layer "F.Cu") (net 3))
 (segment (start 33.19 66.05) (end 35.73 68.59) (width 0.5) (layer "F.Cu") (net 3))
 (segment (start 65.94 39.44) (end 65 38.5) (width 0.5) (layer "F.Cu") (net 3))
 (segment (start 65.94 41.218871) (end 65.94 39.44) (width 0.5) (layer "F.Cu") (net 3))
 (segment (start 30.6625 64.3) (end 30.5 64.4625) (width 0.5) (layer "F.Cu") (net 3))
 (segment (start 33.19 64.3) (end 33.19 66.05) (width 0.5) (layer "F.Cu") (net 3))
 (via (at 65 38.5) (size 0.5) (drill 0.4) (layers "F.Cu" "B.Cu") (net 3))
 (via (at 60.5 29.5) (size 0.5) (drill 0.4) (layers "F.Cu" "B.Cu") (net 3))
 (segment (start 66 43) (end 64.5 44.5) (width 0.5) (layer "B.Cu") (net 3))
 (segment (start 64.5 44.5) (end 49.5 44.5) (width 0.5) (layer "B.Cu") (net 3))
 (segment (start 49.5 44.5) (end 33.19 60.81) (width 0.5) (layer "B.Cu") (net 3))
 (segment (start 33.19 60.81) (end 33.19 64.3) (width 0.5) (layer "B.Cu") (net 3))
 (segment (start 65 38.5) (end 60.5 34) (width 0.5) (layer "B.Cu") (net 3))
 (segment (start 65 38.5) (end 66 39.5) (width 0.5) (layer "B.Cu") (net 3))
 (segment (start 66 39.5) (end 66 43) (width 0.5) (layer "B.Cu") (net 3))
 (segment (start 60.5 34) (end 60.5 29.5) (width 0.5) (layer "B.Cu") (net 3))
 (segment (start 51.97 40.33219) (end 51.97 41.218871) (width 0.25) (layer "F.Cu") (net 7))
 (segment (start 50 37.5) (end 50 38.36219) (width 0.25) (layer "F.Cu") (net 7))
 (segment (start 50.5 37) (end 50 37.5) (width 0.25) (layer "F.Cu") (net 7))
 (segment (start 50 38.36219) (end 51.97 40.33219) (width 0.25) (layer "F.Cu") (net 7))
 (segment (start 49.549 38.549) (end 50.7 39.7) (width 0.25) (layer "F.Cu") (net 5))
 (segment (start 50.7 39.7) (end 50.7 41.218871) (width 0.25) (layer "F.Cu") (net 5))
 (segment (start 48.5 37) (end 49.549 38.049) (width 0.25) (layer "F.Cu") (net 5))
 (segment (start 49.549 38.049) (end 49.549 38.549) (width 0.25) (layer "F.Cu") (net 5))
 (segment (start 51.25 32.25) (end 51 32.5) (width 0.25) (layer "F.Cu") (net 8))
 (segment (start 51.25 28.323872) (end 51.25 32.25) (width 0.25) (layer "F.Cu") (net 8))
 (segment (start 48.25 32.25) (end 48 32.5) (width 0.25) (layer "F.Cu") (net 10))
 (segment (start 48.25 28.323872) (end 48.25 32.25) (width 0.25) (layer "F.Cu") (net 10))
 (segment (start 49.75 28.323872) (end 49.75 34.25) (width 0.25) (layer "F.Cu") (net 6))
 (segment (start 50.493178 29.224872) (end 50.006822 29.224872) (width 0.25) (layer "F.Cu") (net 6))
 (segment (start 49.75 34.25) (end 50.5 35) (width 0.25) (layer "F.Cu") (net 6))
 (segment (start 50.75 28.96805) (end 50.493178 29.224872) (width 0.25) (layer "F.Cu") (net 6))
 (segment (start 50.75 28.323872) (end 50.75 28.96805) (width 0.25) (layer "F.Cu") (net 6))
 (segment (start 49.75 28.96805) (end 49.75 28.323872) (width 0.25) (layer "F.Cu") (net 6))
 (segment (start 50.006822 29.224872) (end 49.75 28.96805) (width 0.25) (layer "F.Cu") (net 6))
 (segment (start 49.993178 27.422872) (end 49.506822 27.422872) (width 0.25) (layer "F.Cu") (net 4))
 (segment (start 49.25 34.25) (end 48.5 35) (width 0.25) (layer "F.Cu") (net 4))
 (segment (start 50.25 28.323872) (end 50.25 27.679694) (width 0.25) (layer "F.Cu") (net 4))
 (segment (start 50.25 27.679694) (end 49.993178 27.422872) (width 0.25) (layer "F.Cu") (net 4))
 (segment (start 49.25 27.679694) (end 49.25 28.323872) (width 0.25) (layer "F.Cu") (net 4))
 (segment (start 49.506822 27.422872) (end 49.25 27.679694) (width 0.25) (layer "F.Cu") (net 4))
 (segment (start 49.25 28.323872) (end 49.25 34.25) (width 0.25) (layer "F.Cu") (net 4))
 (segment (start 35.73 66.59) (end 35.73 64.3) (width 0.25) (layer "F.Cu") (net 12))
 (segment (start 43.5 62.5) (end 47.5 62.5) (width 0.25) (layer "F.Cu") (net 12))
 (segment (start 37.53 62.5) (end 43.5 62.5) (width 0.25) (layer "F.Cu") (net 12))
 (segment (start 35.73 64.3) (end 37.53 62.5) (width 0.25) (layer "F.Cu") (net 12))
 (segment (start 47.5 62.5) (end 50.7 59.3) (width 0.25) (layer "F.Cu") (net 12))
 (segment (start 50.7 59.3) (end 50.7 58.718871) (width 0.25) (layer "F.Cu") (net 12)))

